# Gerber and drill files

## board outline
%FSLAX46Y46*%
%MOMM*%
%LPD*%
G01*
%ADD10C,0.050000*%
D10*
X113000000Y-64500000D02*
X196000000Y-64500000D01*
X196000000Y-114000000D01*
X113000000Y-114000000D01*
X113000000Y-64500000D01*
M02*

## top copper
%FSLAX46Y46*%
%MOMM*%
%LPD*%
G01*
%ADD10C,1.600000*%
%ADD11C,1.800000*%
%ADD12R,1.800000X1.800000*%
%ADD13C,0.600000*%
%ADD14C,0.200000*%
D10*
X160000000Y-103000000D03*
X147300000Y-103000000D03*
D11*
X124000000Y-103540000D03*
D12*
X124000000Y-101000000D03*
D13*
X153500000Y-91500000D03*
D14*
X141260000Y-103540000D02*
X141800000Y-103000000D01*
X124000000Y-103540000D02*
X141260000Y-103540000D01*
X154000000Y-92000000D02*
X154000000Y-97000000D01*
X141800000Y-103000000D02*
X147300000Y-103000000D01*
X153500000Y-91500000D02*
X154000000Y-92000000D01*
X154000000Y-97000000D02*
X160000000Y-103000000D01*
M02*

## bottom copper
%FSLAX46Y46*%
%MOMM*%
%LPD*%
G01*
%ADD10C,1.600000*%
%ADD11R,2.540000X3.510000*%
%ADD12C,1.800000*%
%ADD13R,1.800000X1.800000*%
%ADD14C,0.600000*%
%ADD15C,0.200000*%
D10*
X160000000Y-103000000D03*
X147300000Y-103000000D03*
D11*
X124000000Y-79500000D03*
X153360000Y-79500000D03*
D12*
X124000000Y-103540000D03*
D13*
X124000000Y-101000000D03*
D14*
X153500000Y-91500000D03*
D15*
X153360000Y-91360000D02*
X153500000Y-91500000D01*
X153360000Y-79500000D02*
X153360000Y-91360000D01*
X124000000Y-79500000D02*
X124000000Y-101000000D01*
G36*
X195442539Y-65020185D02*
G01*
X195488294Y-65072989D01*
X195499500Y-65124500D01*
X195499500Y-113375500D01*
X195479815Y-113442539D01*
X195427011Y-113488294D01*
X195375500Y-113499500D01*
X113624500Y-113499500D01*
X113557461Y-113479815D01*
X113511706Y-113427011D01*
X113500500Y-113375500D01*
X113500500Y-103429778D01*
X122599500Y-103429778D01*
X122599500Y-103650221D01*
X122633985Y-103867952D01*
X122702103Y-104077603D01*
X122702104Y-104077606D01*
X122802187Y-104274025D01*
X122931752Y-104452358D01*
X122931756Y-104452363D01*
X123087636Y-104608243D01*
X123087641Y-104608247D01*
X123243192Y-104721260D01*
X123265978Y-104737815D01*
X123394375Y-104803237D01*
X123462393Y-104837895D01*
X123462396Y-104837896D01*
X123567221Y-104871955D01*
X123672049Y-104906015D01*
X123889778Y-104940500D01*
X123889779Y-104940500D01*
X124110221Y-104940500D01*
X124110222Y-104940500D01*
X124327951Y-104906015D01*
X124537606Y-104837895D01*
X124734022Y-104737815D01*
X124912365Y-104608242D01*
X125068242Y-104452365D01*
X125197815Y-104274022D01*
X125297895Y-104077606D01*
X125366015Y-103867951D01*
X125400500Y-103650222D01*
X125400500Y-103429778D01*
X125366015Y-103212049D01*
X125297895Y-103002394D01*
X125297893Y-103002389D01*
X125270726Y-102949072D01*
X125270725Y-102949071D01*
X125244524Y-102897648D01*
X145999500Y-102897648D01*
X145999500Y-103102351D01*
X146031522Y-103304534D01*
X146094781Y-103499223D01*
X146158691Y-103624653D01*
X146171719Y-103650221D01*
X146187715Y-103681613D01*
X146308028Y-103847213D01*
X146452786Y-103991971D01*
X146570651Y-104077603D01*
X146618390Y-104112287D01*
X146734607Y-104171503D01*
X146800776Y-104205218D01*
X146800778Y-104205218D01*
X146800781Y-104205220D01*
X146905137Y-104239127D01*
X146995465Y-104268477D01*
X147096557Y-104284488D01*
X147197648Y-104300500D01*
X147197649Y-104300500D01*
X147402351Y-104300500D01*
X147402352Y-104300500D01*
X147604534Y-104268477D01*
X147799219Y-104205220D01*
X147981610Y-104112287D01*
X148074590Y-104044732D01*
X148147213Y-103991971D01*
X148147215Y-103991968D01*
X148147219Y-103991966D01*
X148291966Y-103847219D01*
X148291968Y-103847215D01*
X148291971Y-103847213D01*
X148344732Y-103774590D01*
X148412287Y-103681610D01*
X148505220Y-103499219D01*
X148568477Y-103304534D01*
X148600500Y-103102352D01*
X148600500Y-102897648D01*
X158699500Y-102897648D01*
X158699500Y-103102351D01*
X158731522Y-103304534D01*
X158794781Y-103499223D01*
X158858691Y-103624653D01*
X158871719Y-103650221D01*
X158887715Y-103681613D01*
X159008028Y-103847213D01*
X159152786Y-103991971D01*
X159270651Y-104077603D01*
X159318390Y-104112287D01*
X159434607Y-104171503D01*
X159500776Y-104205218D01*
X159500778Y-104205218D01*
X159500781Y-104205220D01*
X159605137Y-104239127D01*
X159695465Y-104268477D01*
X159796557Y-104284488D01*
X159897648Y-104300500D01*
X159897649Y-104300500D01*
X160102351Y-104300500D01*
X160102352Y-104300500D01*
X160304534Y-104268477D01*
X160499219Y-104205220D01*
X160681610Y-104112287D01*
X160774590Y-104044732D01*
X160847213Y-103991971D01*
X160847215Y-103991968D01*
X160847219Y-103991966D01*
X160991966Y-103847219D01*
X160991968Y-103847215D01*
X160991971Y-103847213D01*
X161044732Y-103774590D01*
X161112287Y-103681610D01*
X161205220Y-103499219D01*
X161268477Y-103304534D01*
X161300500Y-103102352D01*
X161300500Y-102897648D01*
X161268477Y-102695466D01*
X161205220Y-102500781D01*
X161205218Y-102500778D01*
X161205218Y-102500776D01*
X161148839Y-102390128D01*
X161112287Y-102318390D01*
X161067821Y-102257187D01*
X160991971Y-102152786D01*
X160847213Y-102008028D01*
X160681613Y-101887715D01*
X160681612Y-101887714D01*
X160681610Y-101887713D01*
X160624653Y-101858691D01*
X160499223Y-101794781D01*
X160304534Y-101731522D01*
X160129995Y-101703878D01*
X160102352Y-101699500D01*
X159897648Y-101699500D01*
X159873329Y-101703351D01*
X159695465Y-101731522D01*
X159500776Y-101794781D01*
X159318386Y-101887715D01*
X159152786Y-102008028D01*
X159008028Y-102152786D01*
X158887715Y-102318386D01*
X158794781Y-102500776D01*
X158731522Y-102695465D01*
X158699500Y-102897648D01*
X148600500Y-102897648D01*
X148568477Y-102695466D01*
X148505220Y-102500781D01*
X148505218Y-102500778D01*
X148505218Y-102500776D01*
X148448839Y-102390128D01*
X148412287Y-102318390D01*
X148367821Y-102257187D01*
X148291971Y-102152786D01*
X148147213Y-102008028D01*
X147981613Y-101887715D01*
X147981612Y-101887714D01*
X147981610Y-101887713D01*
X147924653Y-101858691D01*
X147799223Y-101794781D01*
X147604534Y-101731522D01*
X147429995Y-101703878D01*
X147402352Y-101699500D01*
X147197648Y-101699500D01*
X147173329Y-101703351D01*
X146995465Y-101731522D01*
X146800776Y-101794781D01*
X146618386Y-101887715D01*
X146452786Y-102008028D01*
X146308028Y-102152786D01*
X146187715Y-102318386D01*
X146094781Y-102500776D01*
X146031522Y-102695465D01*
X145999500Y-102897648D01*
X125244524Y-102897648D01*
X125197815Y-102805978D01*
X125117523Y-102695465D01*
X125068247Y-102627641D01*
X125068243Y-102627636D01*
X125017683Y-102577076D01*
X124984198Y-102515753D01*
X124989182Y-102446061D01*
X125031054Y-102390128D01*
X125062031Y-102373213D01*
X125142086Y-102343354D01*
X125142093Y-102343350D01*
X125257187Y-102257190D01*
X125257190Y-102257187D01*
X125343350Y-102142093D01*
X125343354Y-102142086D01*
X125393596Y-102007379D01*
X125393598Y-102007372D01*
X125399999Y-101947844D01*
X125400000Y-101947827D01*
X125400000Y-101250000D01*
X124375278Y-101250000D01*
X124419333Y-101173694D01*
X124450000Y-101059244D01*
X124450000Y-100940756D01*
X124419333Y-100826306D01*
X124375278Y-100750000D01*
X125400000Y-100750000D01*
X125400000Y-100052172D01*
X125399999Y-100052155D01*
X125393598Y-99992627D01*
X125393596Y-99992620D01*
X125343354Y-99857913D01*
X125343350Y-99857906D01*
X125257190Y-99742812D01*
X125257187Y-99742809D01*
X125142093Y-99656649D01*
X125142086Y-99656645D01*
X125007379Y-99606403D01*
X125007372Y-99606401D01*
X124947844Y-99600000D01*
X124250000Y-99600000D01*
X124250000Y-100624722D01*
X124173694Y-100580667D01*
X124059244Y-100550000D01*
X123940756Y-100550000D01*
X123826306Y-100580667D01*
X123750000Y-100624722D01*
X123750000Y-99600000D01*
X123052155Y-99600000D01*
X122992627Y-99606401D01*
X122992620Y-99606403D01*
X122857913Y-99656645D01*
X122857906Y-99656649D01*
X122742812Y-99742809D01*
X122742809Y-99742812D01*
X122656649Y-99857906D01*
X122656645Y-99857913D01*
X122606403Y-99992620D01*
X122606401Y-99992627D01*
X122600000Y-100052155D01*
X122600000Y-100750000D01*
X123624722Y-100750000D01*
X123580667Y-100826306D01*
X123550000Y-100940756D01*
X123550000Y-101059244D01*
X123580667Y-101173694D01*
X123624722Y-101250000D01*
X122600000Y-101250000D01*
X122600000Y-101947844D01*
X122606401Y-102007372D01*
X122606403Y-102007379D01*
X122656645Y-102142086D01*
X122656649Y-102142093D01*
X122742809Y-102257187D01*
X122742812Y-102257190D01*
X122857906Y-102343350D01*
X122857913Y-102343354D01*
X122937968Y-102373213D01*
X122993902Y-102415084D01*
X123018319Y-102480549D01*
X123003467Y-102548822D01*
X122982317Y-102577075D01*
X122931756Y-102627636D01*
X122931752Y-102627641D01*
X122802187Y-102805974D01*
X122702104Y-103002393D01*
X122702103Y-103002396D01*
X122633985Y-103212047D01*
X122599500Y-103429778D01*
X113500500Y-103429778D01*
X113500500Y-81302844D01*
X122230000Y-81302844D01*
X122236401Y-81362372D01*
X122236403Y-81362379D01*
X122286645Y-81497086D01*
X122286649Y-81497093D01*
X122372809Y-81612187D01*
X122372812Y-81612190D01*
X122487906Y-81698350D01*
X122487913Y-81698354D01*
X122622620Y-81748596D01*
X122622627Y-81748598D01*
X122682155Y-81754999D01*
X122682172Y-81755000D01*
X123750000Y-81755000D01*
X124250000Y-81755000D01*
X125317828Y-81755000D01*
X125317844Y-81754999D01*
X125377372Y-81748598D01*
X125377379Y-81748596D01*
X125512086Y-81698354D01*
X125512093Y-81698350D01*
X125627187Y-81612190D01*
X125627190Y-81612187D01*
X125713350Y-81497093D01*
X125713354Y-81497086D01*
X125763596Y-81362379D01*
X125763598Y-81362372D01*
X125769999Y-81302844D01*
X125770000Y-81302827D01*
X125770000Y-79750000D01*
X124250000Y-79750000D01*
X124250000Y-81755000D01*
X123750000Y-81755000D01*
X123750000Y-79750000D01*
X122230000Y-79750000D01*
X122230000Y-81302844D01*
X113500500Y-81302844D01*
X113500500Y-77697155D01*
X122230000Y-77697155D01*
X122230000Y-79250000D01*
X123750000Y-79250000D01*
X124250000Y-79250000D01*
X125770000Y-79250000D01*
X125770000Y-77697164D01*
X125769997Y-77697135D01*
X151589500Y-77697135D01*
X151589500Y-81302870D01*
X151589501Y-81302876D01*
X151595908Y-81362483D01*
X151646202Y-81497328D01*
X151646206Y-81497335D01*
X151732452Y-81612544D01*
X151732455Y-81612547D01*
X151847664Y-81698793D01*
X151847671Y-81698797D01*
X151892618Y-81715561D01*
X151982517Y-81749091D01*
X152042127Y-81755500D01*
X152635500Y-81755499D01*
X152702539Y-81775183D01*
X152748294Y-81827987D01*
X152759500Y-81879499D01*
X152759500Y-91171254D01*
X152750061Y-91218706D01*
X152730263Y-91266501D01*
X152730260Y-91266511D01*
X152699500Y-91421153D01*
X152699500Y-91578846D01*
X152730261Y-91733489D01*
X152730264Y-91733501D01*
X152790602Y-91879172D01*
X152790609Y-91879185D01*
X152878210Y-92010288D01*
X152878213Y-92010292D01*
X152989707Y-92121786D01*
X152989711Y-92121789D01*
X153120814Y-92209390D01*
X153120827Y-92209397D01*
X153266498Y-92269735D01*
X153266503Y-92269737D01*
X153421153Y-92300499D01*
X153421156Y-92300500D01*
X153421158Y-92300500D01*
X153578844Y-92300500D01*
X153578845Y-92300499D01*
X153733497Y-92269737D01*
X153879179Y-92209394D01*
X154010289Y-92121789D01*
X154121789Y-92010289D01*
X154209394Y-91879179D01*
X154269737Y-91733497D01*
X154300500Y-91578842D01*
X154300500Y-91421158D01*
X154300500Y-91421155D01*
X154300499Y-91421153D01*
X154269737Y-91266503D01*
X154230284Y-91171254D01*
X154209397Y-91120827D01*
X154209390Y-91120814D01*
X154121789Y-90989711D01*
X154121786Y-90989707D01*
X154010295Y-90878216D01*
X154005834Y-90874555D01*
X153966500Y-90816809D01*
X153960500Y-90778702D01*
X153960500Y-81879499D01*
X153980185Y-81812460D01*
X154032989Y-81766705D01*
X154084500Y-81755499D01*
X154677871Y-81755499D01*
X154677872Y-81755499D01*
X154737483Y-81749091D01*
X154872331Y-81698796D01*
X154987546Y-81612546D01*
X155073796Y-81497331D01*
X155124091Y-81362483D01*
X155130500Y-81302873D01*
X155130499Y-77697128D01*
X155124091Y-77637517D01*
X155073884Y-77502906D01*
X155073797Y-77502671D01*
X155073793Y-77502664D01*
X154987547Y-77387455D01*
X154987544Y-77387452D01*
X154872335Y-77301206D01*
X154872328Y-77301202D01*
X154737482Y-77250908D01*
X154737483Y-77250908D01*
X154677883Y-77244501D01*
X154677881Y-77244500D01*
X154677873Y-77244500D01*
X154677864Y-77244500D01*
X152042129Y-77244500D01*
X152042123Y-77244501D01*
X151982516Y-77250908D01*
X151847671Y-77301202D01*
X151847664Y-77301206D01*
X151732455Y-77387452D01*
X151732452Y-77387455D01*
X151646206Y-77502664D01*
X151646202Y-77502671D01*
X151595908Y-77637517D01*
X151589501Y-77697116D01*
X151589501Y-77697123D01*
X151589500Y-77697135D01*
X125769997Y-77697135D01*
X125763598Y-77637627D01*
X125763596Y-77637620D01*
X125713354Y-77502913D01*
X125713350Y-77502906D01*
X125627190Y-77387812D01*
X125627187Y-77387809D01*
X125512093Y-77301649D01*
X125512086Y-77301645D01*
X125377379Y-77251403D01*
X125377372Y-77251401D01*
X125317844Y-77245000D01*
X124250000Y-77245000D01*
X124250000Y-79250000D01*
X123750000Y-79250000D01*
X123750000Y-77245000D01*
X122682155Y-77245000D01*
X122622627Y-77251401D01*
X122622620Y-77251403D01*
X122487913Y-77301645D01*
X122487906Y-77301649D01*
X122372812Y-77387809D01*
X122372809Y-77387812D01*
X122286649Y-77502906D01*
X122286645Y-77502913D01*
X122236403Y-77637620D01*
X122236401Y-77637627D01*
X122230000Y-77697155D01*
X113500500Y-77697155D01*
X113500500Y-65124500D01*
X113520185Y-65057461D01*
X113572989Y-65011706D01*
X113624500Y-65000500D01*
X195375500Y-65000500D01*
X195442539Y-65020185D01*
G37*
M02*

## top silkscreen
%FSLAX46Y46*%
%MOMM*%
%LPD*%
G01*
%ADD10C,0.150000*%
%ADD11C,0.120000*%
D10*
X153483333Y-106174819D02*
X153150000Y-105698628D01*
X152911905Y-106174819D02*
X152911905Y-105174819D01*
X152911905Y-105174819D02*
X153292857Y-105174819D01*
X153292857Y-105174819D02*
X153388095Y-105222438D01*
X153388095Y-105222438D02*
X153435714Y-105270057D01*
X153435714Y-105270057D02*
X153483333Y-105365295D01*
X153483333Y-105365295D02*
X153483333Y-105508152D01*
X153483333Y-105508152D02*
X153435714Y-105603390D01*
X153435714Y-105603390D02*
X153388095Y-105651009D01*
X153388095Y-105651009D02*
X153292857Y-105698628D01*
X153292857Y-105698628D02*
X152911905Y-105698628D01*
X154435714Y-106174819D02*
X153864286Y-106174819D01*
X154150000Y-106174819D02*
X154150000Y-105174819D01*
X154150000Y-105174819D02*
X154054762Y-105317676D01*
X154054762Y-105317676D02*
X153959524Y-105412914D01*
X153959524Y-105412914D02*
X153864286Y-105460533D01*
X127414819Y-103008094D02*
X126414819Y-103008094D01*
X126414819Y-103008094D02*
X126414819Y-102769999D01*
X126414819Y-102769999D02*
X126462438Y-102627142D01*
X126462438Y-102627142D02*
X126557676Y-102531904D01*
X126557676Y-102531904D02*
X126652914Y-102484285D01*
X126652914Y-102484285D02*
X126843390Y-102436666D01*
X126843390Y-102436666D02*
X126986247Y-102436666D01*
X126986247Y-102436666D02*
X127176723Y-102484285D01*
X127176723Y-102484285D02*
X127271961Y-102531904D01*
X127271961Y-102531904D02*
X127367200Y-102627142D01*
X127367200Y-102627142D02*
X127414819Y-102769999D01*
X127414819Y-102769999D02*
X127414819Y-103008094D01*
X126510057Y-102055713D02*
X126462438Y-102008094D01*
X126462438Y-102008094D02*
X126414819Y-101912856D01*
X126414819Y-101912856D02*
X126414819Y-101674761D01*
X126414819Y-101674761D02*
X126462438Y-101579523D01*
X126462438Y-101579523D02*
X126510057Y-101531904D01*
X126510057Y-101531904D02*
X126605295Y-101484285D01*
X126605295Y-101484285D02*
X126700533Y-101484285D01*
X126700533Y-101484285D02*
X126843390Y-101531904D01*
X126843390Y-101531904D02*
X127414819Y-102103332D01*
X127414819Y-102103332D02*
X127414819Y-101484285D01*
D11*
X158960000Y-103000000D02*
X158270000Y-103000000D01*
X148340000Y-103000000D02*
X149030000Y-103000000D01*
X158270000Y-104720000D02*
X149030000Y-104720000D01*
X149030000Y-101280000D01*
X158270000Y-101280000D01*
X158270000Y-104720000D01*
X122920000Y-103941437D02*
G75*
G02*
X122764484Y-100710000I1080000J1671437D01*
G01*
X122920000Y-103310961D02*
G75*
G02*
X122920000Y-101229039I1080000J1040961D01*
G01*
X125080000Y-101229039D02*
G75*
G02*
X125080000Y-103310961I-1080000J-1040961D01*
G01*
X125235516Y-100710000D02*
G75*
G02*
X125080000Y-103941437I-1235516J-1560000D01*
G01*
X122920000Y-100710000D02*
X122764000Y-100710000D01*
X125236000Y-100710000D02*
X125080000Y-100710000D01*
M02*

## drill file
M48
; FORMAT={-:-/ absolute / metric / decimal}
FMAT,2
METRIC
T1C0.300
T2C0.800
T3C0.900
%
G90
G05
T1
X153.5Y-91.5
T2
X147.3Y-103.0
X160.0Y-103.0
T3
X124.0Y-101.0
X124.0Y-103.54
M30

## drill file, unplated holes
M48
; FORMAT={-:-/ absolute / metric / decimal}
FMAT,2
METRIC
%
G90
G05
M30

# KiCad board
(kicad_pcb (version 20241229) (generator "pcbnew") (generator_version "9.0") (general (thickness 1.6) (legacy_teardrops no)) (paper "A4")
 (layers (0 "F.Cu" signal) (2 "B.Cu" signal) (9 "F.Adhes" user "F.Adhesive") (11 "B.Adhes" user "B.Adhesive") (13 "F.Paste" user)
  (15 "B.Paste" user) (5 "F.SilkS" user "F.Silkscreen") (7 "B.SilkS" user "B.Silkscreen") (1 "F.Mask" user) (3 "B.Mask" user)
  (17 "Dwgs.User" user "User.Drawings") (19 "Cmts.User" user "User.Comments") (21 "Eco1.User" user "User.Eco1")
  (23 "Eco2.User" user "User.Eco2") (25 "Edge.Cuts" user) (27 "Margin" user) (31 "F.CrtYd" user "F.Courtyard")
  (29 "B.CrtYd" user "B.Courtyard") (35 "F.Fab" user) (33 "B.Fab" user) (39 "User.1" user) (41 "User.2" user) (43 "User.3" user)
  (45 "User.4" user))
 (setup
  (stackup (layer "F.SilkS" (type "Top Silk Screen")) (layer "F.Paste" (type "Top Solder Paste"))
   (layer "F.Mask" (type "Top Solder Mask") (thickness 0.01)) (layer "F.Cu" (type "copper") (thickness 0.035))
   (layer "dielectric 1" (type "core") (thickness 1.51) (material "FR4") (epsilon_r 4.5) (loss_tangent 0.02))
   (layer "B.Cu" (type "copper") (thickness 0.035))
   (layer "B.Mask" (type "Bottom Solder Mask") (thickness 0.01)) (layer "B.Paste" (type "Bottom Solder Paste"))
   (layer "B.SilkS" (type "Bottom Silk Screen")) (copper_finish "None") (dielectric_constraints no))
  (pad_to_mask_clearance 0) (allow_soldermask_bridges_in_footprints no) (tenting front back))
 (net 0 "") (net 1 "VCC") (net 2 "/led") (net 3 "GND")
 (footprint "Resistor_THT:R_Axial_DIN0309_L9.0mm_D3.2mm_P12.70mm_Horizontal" (layer "F.Cu") (at 160 103 180)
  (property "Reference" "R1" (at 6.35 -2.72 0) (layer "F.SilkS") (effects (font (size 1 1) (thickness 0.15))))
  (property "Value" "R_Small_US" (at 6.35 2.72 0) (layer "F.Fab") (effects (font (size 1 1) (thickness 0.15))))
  (fp_line (start 11.66 0) (end 10.97 0) (stroke (width 0.12) (type solid)) (layer "F.SilkS"))
  (fp_line (start 1.04 0) (end 1.73 0) (stroke (width 0.12) (type solid)) (layer "F.SilkS"))
  (fp_rect (start 1.73 -1.72) (end 10.97 1.72) (stroke (width 0.12) (type solid)) (fill no) (layer "F.SilkS"))
  (pad "1" thru_hole circle (at 0 0 180) (size 1.6 1.6) (drill 0.8) (layers "*.Cu" "*.Mask") (remove_unused_layers no) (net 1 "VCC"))
  (pad "2" thru_hole circle (at 12.7 0 180) (size 1.6 1.6) (drill 0.8) (layers "*.Cu" "*.Mask") (remove_unused_layers no) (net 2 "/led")))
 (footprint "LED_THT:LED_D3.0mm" (layer "F.Cu") (at 124 101 -90)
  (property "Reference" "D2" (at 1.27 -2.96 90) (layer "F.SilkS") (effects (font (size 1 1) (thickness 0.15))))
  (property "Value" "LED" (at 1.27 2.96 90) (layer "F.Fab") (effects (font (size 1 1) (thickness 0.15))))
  (fp_line (start -0.29 1.08) (end -0.29 1.236) (stroke (width 0.12) (type solid)) (layer "F.SilkS"))
  (fp_line (start -0.29 -1.236) (end -0.29 -1.08) (stroke (width 0.12) (type solid)) (layer "F.SilkS"))
  (fp_arc (start 2.310961 1.08) (mid 1.27 1.5) (end 0.229039 1.08) (stroke (width 0.12) (type solid)) (layer "F.SilkS"))
  (fp_arc (start 2.941437 1.08) (mid 1.36566 1.987699) (end -0.29 1.235516) (stroke (width 0.12) (type solid)) (layer "F.SilkS"))
  (fp_arc (start 0.229039 -1.08) (mid 1.27 -1.5) (end 2.310961 -1.08) (stroke (width 0.12) (type solid)) (layer "F.SilkS"))
  (fp_arc (start -0.29 -1.235516) (mid 1.36566 -1.987699) (end 2.941437 -1.08) (stroke (width 0.12) (type solid)) (layer "F.SilkS"))
  (pad "1" thru_hole rect (at 0 0 270) (size 1.8 1.8) (drill 0.9) (layers "*.Cu" "*.Mask") (remove_unused_layers no) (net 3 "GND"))
  (pad "2" thru_hole circle (at 2.54 0 270) (size 1.8 1.8) (drill 0.9) (layers "*.Cu" "*.Mask") (remove_unused_layers no) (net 2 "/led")))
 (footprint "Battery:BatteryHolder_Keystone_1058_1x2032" (layer "B.Cu") (at 138.68 79.5 180)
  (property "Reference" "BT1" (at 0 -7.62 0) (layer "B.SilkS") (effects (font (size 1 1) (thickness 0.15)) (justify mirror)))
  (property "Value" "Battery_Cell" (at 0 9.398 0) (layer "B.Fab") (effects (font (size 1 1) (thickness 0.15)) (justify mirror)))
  (pad "1" smd rect (at -14.68 0 180) (size 2.54 3.51) (layers "B.Cu" "B.Mask" "B.Paste") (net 1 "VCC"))
  (pad "2" smd rect (at 14.68 0 180) (size 2.54 3.51) (layers "B.Cu" "B.Mask" "B.Paste") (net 3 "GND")))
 (gr_rect (start 113 64.5) (end 196 114) (stroke (width 0.05) (type default)) (fill no) (layer "Edge.Cuts"))
 (segment (start 154 92) (end 154 97) (width 0.2) (layer "F.Cu") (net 1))
 (segment (start 154 97) (end 160 103) (width 0.2) (layer "F.Cu") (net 1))
 (segment (start 153.5 91.5) (end 154 92) (width 0.2) (layer "F.Cu") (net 1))
 (via (at 153.5 91.5) (size 0.6) (drill 0.3) (layers "F.Cu" "B.Cu") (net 1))
 (segment (start 153.36 79.5) (end 153.36 91.36) (width 0.2) (layer "B.Cu") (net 1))
 (segment (start 153.36 91.36) (end 153.5 91.5) (width 0.2) (layer "B.Cu") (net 1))
 (segment (start 124 79.5) (end 124 101) (width 0.2) (layer "B.Cu") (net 3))
 (segment (start 124 103.54) (end 141.26 103.54) (width 0.2) (layer "F.Cu") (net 2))
 (segment (start 141.8 103) (end 147.3 103) (width 0.2) (layer "F.Cu") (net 2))
 (segment (start 141.26 103.54) (end 141.8 103) (width 0.2) (layer "F.Cu") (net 2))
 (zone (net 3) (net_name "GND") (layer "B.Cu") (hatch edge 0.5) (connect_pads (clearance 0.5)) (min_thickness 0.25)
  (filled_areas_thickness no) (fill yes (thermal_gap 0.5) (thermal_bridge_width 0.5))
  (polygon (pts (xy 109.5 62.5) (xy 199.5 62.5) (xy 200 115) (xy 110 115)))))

